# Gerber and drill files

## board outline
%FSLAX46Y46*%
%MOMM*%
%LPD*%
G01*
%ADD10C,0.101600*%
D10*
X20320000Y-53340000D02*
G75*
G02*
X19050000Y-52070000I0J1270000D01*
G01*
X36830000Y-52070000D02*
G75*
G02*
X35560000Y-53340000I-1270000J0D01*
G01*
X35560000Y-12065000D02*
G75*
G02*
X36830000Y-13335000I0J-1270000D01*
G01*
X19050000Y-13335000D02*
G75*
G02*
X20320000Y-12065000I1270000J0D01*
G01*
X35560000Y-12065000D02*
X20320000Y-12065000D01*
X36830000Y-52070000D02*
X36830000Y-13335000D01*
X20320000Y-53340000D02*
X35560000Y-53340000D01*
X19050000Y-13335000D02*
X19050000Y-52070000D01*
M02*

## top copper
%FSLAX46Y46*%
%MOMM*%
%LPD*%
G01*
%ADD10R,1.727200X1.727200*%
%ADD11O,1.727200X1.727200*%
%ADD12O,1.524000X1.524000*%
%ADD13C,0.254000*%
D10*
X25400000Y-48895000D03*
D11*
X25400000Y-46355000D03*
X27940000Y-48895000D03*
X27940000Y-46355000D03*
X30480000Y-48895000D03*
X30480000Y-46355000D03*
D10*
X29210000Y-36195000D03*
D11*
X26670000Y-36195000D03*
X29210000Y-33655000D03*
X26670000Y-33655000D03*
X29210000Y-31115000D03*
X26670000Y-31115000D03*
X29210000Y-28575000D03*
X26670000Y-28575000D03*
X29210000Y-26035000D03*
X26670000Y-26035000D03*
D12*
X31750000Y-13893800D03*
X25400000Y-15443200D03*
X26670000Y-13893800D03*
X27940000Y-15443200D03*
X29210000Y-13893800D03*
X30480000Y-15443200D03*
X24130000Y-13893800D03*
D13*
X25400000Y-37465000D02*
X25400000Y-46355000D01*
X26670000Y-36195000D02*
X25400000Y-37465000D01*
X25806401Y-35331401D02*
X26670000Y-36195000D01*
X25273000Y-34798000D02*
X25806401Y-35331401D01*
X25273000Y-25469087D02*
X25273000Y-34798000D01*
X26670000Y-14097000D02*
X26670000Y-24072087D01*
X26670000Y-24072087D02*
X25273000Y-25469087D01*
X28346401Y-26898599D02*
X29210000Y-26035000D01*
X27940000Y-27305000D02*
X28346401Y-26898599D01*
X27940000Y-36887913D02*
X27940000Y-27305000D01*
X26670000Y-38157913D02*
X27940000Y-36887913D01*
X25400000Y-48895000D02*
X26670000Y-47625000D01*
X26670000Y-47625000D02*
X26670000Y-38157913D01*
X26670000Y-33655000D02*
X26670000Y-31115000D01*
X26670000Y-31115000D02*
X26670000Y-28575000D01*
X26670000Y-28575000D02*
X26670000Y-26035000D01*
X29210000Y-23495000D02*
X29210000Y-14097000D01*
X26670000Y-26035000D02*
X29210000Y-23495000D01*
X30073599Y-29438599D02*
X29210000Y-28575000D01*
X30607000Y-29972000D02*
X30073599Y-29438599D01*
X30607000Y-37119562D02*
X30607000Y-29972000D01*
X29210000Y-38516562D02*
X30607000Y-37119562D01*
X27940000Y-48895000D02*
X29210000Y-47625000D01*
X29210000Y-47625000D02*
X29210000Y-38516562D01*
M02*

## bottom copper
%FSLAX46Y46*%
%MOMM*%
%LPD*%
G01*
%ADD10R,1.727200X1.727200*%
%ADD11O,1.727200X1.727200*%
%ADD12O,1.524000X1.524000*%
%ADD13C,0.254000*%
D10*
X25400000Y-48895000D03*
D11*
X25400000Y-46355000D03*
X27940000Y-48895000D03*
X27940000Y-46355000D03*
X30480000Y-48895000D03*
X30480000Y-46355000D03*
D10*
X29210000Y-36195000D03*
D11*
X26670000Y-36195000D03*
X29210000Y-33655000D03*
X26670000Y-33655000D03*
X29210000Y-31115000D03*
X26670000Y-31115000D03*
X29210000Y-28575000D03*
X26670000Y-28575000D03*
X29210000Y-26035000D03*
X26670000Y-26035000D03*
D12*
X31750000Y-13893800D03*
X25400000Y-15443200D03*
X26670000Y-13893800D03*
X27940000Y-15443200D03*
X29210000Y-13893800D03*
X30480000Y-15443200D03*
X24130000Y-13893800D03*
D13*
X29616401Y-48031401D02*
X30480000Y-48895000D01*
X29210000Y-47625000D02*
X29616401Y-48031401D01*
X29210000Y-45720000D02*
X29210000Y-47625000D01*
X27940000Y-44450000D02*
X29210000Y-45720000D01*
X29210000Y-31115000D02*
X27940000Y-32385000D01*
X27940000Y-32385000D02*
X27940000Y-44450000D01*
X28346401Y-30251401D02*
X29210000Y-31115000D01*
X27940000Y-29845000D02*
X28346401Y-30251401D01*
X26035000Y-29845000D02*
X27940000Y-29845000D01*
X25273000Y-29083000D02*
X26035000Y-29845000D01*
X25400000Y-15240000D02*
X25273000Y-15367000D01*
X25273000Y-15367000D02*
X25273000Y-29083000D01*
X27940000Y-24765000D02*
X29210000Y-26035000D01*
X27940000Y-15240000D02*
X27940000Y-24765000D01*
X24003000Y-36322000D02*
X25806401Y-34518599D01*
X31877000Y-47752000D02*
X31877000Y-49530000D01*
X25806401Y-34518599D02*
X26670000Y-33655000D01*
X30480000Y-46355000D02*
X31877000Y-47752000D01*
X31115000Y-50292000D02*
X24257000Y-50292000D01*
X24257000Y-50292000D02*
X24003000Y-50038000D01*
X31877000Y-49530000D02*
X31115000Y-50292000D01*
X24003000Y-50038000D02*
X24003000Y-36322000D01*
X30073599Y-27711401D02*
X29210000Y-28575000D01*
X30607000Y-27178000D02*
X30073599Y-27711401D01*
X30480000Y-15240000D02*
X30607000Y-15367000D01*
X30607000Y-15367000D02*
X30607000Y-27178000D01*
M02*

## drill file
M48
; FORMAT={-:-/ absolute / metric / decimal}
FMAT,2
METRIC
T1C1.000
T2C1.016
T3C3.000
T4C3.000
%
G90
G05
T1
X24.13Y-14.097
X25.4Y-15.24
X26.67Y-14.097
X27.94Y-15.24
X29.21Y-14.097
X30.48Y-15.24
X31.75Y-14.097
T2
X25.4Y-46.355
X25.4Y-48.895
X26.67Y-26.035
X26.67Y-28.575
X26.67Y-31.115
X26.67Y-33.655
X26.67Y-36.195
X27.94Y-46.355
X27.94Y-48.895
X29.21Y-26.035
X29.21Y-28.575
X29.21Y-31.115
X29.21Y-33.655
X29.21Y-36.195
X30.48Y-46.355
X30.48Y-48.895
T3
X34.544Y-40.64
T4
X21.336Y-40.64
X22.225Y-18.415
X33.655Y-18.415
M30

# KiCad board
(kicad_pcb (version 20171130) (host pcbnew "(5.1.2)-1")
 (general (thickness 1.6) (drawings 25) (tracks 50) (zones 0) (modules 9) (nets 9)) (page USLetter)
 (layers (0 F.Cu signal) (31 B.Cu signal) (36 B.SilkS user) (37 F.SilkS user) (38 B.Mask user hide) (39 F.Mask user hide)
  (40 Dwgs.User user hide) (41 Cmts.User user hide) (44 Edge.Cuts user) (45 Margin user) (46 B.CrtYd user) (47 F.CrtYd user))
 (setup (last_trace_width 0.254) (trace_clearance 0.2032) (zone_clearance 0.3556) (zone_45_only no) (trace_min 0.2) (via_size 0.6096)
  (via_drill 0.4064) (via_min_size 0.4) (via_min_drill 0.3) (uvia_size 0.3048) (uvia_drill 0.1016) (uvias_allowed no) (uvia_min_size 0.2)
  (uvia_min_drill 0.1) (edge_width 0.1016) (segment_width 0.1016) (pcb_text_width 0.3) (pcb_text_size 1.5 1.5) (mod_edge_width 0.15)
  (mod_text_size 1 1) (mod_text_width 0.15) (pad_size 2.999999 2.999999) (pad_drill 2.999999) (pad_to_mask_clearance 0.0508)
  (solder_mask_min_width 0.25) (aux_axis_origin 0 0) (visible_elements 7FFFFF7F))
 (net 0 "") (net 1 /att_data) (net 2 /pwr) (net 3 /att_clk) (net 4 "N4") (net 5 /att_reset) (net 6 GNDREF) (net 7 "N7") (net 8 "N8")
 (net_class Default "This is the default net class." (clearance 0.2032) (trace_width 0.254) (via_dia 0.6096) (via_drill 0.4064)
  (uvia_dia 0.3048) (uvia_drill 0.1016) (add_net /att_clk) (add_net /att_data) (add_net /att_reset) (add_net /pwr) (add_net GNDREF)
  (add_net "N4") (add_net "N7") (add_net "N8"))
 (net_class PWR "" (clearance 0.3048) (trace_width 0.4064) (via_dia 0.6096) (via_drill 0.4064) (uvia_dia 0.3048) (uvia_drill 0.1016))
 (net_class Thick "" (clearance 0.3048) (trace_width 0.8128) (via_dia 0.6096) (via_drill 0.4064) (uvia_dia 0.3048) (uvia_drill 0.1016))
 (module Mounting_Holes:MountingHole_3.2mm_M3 (layer F.Cu) (at 34.544 40.64)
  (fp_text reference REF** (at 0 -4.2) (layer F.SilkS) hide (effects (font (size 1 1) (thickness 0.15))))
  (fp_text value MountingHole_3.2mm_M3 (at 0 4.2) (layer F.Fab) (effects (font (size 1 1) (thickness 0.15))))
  (pad "" np_thru_hole circle (at 0 0) (size 2.999999 2.999999) (drill 2.999999) (layers *.Cu *.Mask)))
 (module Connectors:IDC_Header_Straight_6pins (layer F.Cu) (at 25.4 48.895)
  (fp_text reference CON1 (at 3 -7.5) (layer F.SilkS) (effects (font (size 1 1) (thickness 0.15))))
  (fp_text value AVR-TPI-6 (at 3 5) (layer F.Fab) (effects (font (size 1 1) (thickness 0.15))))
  (pad 1 thru_hole rect (at 0 0) (size 1.7272 1.7272) (drill 1.016) (layers *.Cu *.Mask) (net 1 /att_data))
  (pad 2 thru_hole oval (at 0 -2.54) (size 1.7272 1.7272) (drill 1.016) (layers *.Cu *.Mask) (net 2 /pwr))
  (pad 3 thru_hole oval (at 2.54 0) (size 1.7272 1.7272) (drill 1.016) (layers *.Cu *.Mask) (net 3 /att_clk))
  (pad 4 thru_hole oval (at 2.54 -2.54) (size 1.7272 1.7272) (drill 1.016) (layers *.Cu *.Mask) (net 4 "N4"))
  (pad 5 thru_hole oval (at 5.08 0) (size 1.7272 1.7272) (drill 1.016) (layers *.Cu *.Mask) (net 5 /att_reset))
  (pad 6 thru_hole oval (at 5.08 -2.54) (size 1.7272 1.7272) (drill 1.016) (layers *.Cu *.Mask) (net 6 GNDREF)))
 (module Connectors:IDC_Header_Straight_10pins (layer F.Cu) (at 29.21 36.195 90)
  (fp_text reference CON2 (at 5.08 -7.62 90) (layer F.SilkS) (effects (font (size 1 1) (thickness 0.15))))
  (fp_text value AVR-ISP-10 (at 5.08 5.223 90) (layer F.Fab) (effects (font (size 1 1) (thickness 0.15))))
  (pad 1 thru_hole rect (at 0 0 90) (size 1.7272 1.7272) (drill 1.016) (layers *.Cu *.Mask) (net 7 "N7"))
  (pad 2 thru_hole oval (at 0 -2.54 90) (size 1.7272 1.7272) (drill 1.016) (layers *.Cu *.Mask) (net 2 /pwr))
  (pad 3 thru_hole oval (at 2.54 0 90) (size 1.7272 1.7272) (drill 1.016) (layers *.Cu *.Mask) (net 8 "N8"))
  (pad 4 thru_hole oval (at 2.54 -2.54 90) (size 1.7272 1.7272) (drill 1.016) (layers *.Cu *.Mask) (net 6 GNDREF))
  (pad 5 thru_hole oval (at 5.08 0 90) (size 1.7272 1.7272) (drill 1.016) (layers *.Cu *.Mask) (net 5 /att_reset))
  (pad 6 thru_hole oval (at 5.08 -2.54 90) (size 1.7272 1.7272) (drill 1.016) (layers *.Cu *.Mask) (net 6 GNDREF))
  (pad 7 thru_hole oval (at 7.62 0 90) (size 1.7272 1.7272) (drill 1.016) (layers *.Cu *.Mask) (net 3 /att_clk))
  (pad 8 thru_hole oval (at 7.62 -2.54 90) (size 1.7272 1.7272) (drill 1.016) (layers *.Cu *.Mask) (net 6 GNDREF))
  (pad 9 thru_hole oval (at 10.16 0 90) (size 1.7272 1.7272) (drill 1.016) (layers *.Cu *.Mask) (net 1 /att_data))
  (pad 10 thru_hole oval (at 10.16 -2.54 90) (size 1.7272 1.7272) (drill 1.016) (layers *.Cu *.Mask) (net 6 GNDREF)))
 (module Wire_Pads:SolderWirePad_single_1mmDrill (layer F.Cu) (at 29.845 14.351 90)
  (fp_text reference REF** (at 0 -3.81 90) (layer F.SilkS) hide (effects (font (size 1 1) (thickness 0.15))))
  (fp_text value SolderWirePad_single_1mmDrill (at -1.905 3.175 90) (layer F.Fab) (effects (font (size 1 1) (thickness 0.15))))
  (pad 1 thru_hole oval (at 0.254 1.905 90) (size 1.524 1.524) (drill 1 (offset 0.2032 0)) (layers *.Cu *.Mask)))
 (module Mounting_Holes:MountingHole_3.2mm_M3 (layer F.Cu) (at 33.655 18.415)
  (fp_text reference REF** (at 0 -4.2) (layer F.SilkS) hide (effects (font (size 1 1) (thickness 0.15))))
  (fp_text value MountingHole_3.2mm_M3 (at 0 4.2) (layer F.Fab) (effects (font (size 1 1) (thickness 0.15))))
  (pad "" np_thru_hole circle (at 0 0) (size 3 3) (drill 3) (layers *.Cu *.Mask)))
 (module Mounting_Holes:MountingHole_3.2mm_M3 (layer F.Cu) (at 21.336 40.64)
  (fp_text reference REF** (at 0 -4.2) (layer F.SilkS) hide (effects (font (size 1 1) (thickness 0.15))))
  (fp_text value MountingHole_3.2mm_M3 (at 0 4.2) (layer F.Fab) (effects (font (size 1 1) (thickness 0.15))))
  (pad "" np_thru_hole circle (at 0 0) (size 3 3) (drill 3) (layers *.Cu *.Mask)))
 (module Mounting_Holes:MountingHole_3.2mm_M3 (layer F.Cu) (at 22.225 18.415)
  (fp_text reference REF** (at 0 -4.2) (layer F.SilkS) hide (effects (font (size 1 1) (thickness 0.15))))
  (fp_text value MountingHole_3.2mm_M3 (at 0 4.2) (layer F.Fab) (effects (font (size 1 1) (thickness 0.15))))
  (pad "" np_thru_hole circle (at 0 0) (size 3 3) (drill 3) (layers *.Cu *.Mask)))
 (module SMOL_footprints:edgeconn (layer F.Cu) (at 25.4 14.605 90)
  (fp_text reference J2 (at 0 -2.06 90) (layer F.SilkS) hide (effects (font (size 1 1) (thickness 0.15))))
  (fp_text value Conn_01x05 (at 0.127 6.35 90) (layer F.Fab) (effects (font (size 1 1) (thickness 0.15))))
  (pad 1 thru_hole oval (at -0.635 0 90) (size 1.524 1.524) (drill 1 (offset -0.2032 0)) (layers *.Cu *.Mask) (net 5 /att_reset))
  (pad 2 thru_hole oval (at 0.508 1.27 90) (size 1.524 1.524) (drill 1 (offset 0.2032 0)) (layers *.Cu *.Mask) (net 2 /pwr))
  (pad 3 thru_hole oval (at -0.635 2.54 90) (size 1.524 1.524) (drill 1 (offset -0.2032 0)) (layers *.Cu *.Mask) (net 1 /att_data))
  (pad 4 thru_hole oval (at 0.508 3.81 90) (size 1.524 1.524) (drill 1 (offset 0.2032 0)) (layers *.Cu *.Mask) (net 6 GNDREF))
  (pad 5 thru_hole oval (at -0.635 5.08 90) (size 1.524 1.524) (drill 1 (offset -0.2032 0)) (layers *.Cu *.Mask) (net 3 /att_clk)))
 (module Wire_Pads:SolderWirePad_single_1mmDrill (layer F.Cu) (at 22.225 14.351 90)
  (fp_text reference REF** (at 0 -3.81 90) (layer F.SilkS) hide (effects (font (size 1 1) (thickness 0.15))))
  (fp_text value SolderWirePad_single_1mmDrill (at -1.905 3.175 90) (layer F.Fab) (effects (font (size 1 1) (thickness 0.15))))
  (pad 1 thru_hole oval (at 0.254 1.905 90) (size 1.524 1.524) (drill 1 (offset 0.2032 0)) (layers *.Cu *.Mask)))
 (gr_arc (start 20.32 52.07) (end 19.05 52.07) (angle -90) (layer Edge.Cuts) (width 0.1016))
 (gr_arc (start 35.56 52.07) (end 35.56 53.34) (angle -90) (layer Edge.Cuts) (width 0.1016))
 (gr_arc (start 35.56 13.335) (end 36.83 13.335) (angle -90) (layer Edge.Cuts) (width 0.1016))
 (gr_arc (start 20.32 13.335) (end 20.32 12.065) (angle -90) (layer Edge.Cuts) (width 0.1016))
 (gr_line (start 35.56 12.065) (end 20.32 12.065) (layer Edge.Cuts) (width 0.1016))
 (gr_line (start 36.83 52.07) (end 36.83 13.335) (layer Edge.Cuts) (width 0.1016))
 (gr_line (start 20.32 53.34) (end 35.56 53.34) (layer Edge.Cuts) (width 0.1016))
 (gr_line (start 19.05 13.335) (end 19.05 52.07) (layer Edge.Cuts) (width 0.1016))
 (segment (start 25.4 37.465) (end 25.4 46.355) (width 0.254) (layer F.Cu) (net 2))
 (segment (start 26.67 36.195) (end 25.4 37.465) (width 0.254) (layer F.Cu) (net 2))
 (segment (start 25.806401 35.331401) (end 26.67 36.195) (width 0.254) (layer F.Cu) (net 2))
 (segment (start 25.273 34.798) (end 25.806401 35.331401) (width 0.254) (layer F.Cu) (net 2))
 (segment (start 25.273 25.469087) (end 25.273 34.798) (width 0.254) (layer F.Cu) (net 2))
 (segment (start 26.67 14.097) (end 26.67 24.072087) (width 0.254) (layer F.Cu) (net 2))
 (segment (start 26.67 24.072087) (end 25.273 25.469087) (width 0.254) (layer F.Cu) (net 2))
 (segment (start 29.616401 48.031401) (end 30.48 48.895) (width 0.254) (layer B.Cu) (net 5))
 (segment (start 29.21 47.625) (end 29.616401 48.031401) (width 0.254) (layer B.Cu) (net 5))
 (segment (start 29.21 45.72) (end 29.21 47.625) (width 0.254) (layer B.Cu) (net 5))
 (segment (start 27.94 44.45) (end 29.21 45.72) (width 0.254) (layer B.Cu) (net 5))
 (segment (start 29.21 31.115) (end 27.94 32.385) (width 0.254) (layer B.Cu) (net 5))
 (segment (start 27.94 32.385) (end 27.94 44.45) (width 0.254) (layer B.Cu) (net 5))
 (segment (start 28.346401 30.251401) (end 29.21 31.115) (width 0.254) (layer B.Cu) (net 5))
 (segment (start 27.94 29.845) (end 28.346401 30.251401) (width 0.254) (layer B.Cu) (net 5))
 (segment (start 26.035 29.845) (end 27.94 29.845) (width 0.254) (layer B.Cu) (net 5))
 (segment (start 25.273 29.083) (end 26.035 29.845) (width 0.254) (layer B.Cu) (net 5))
 (segment (start 25.4 15.24) (end 25.273 15.367) (width 0.254) (layer B.Cu) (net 5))
 (segment (start 25.273 15.367) (end 25.273 29.083) (width 0.254) (layer B.Cu) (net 5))
 (segment (start 27.94 24.765) (end 29.21 26.035) (width 0.254) (layer B.Cu) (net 1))
 (segment (start 27.94 15.24) (end 27.94 24.765) (width 0.254) (layer B.Cu) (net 1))
 (segment (start 28.346401 26.898599) (end 29.21 26.035) (width 0.254) (layer F.Cu) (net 1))
 (segment (start 27.94 27.305) (end 28.346401 26.898599) (width 0.254) (layer F.Cu) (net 1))
 (segment (start 27.94 36.887913) (end 27.94 27.305) (width 0.254) (layer F.Cu) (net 1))
 (segment (start 26.67 38.157913) (end 27.94 36.887913) (width 0.254) (layer F.Cu) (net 1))
 (segment (start 25.4 48.895) (end 26.67 47.625) (width 0.254) (layer F.Cu) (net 1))
 (segment (start 26.67 47.625) (end 26.67 38.157913) (width 0.254) (layer F.Cu) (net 1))
 (segment (start 26.67 33.655) (end 26.67 31.115) (width 0.254) (layer F.Cu) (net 6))
 (segment (start 26.67 31.115) (end 26.67 28.575) (width 0.254) (layer F.Cu) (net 6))
 (segment (start 26.67 28.575) (end 26.67 26.035) (width 0.254) (layer F.Cu) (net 6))
 (segment (start 29.21 23.495) (end 29.21 14.097) (width 0.254) (layer F.Cu) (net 6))
 (segment (start 26.67 26.035) (end 29.21 23.495) (width 0.254) (layer F.Cu) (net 6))
 (segment (start 24.003 36.322) (end 25.806401 34.518599) (width 0.254) (layer B.Cu) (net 6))
 (segment (start 31.877 47.752) (end 31.877 49.53) (width 0.254) (layer B.Cu) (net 6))
 (segment (start 25.806401 34.518599) (end 26.67 33.655) (width 0.254) (layer B.Cu) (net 6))
 (segment (start 30.48 46.355) (end 31.877 47.752) (width 0.254) (layer B.Cu) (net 6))
 (segment (start 31.115 50.292) (end 24.257 50.292) (width 0.254) (layer B.Cu) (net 6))
 (segment (start 24.257 50.292) (end 24.003 50.038) (width 0.254) (layer B.Cu) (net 6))
 (segment (start 31.877 49.53) (end 31.115 50.292) (width 0.254) (layer B.Cu) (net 6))
 (segment (start 24.003 50.038) (end 24.003 36.322) (width 0.254) (layer B.Cu) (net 6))
 (segment (start 30.073599 29.438599) (end 29.21 28.575) (width 0.254) (layer F.Cu) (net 3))
 (segment (start 30.607 29.972) (end 30.073599 29.438599) (width 0.254) (layer F.Cu) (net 3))
 (segment (start 30.607 37.119562) (end 30.607 29.972) (width 0.254) (layer F.Cu) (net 3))
 (segment (start 29.21 38.516562) (end 30.607 37.119562) (width 0.254) (layer F.Cu) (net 3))
 (segment (start 27.94 48.895) (end 29.21 47.625) (width 0.254) (layer F.Cu) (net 3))
 (segment (start 29.21 47.625) (end 29.21 38.516562) (width 0.254) (layer F.Cu) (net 3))
 (segment (start 30.073599 27.711401) (end 29.21 28.575) (width 0.254) (layer B.Cu) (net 3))
 (segment (start 30.607 27.178) (end 30.073599 27.711401) (width 0.254) (layer B.Cu) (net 3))
 (segment (start 30.48 15.24) (end 30.607 15.367) (width 0.254) (layer B.Cu) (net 3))
 (segment (start 30.607 15.367) (end 30.607 27.178) (width 0.254) (layer B.Cu) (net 3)))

